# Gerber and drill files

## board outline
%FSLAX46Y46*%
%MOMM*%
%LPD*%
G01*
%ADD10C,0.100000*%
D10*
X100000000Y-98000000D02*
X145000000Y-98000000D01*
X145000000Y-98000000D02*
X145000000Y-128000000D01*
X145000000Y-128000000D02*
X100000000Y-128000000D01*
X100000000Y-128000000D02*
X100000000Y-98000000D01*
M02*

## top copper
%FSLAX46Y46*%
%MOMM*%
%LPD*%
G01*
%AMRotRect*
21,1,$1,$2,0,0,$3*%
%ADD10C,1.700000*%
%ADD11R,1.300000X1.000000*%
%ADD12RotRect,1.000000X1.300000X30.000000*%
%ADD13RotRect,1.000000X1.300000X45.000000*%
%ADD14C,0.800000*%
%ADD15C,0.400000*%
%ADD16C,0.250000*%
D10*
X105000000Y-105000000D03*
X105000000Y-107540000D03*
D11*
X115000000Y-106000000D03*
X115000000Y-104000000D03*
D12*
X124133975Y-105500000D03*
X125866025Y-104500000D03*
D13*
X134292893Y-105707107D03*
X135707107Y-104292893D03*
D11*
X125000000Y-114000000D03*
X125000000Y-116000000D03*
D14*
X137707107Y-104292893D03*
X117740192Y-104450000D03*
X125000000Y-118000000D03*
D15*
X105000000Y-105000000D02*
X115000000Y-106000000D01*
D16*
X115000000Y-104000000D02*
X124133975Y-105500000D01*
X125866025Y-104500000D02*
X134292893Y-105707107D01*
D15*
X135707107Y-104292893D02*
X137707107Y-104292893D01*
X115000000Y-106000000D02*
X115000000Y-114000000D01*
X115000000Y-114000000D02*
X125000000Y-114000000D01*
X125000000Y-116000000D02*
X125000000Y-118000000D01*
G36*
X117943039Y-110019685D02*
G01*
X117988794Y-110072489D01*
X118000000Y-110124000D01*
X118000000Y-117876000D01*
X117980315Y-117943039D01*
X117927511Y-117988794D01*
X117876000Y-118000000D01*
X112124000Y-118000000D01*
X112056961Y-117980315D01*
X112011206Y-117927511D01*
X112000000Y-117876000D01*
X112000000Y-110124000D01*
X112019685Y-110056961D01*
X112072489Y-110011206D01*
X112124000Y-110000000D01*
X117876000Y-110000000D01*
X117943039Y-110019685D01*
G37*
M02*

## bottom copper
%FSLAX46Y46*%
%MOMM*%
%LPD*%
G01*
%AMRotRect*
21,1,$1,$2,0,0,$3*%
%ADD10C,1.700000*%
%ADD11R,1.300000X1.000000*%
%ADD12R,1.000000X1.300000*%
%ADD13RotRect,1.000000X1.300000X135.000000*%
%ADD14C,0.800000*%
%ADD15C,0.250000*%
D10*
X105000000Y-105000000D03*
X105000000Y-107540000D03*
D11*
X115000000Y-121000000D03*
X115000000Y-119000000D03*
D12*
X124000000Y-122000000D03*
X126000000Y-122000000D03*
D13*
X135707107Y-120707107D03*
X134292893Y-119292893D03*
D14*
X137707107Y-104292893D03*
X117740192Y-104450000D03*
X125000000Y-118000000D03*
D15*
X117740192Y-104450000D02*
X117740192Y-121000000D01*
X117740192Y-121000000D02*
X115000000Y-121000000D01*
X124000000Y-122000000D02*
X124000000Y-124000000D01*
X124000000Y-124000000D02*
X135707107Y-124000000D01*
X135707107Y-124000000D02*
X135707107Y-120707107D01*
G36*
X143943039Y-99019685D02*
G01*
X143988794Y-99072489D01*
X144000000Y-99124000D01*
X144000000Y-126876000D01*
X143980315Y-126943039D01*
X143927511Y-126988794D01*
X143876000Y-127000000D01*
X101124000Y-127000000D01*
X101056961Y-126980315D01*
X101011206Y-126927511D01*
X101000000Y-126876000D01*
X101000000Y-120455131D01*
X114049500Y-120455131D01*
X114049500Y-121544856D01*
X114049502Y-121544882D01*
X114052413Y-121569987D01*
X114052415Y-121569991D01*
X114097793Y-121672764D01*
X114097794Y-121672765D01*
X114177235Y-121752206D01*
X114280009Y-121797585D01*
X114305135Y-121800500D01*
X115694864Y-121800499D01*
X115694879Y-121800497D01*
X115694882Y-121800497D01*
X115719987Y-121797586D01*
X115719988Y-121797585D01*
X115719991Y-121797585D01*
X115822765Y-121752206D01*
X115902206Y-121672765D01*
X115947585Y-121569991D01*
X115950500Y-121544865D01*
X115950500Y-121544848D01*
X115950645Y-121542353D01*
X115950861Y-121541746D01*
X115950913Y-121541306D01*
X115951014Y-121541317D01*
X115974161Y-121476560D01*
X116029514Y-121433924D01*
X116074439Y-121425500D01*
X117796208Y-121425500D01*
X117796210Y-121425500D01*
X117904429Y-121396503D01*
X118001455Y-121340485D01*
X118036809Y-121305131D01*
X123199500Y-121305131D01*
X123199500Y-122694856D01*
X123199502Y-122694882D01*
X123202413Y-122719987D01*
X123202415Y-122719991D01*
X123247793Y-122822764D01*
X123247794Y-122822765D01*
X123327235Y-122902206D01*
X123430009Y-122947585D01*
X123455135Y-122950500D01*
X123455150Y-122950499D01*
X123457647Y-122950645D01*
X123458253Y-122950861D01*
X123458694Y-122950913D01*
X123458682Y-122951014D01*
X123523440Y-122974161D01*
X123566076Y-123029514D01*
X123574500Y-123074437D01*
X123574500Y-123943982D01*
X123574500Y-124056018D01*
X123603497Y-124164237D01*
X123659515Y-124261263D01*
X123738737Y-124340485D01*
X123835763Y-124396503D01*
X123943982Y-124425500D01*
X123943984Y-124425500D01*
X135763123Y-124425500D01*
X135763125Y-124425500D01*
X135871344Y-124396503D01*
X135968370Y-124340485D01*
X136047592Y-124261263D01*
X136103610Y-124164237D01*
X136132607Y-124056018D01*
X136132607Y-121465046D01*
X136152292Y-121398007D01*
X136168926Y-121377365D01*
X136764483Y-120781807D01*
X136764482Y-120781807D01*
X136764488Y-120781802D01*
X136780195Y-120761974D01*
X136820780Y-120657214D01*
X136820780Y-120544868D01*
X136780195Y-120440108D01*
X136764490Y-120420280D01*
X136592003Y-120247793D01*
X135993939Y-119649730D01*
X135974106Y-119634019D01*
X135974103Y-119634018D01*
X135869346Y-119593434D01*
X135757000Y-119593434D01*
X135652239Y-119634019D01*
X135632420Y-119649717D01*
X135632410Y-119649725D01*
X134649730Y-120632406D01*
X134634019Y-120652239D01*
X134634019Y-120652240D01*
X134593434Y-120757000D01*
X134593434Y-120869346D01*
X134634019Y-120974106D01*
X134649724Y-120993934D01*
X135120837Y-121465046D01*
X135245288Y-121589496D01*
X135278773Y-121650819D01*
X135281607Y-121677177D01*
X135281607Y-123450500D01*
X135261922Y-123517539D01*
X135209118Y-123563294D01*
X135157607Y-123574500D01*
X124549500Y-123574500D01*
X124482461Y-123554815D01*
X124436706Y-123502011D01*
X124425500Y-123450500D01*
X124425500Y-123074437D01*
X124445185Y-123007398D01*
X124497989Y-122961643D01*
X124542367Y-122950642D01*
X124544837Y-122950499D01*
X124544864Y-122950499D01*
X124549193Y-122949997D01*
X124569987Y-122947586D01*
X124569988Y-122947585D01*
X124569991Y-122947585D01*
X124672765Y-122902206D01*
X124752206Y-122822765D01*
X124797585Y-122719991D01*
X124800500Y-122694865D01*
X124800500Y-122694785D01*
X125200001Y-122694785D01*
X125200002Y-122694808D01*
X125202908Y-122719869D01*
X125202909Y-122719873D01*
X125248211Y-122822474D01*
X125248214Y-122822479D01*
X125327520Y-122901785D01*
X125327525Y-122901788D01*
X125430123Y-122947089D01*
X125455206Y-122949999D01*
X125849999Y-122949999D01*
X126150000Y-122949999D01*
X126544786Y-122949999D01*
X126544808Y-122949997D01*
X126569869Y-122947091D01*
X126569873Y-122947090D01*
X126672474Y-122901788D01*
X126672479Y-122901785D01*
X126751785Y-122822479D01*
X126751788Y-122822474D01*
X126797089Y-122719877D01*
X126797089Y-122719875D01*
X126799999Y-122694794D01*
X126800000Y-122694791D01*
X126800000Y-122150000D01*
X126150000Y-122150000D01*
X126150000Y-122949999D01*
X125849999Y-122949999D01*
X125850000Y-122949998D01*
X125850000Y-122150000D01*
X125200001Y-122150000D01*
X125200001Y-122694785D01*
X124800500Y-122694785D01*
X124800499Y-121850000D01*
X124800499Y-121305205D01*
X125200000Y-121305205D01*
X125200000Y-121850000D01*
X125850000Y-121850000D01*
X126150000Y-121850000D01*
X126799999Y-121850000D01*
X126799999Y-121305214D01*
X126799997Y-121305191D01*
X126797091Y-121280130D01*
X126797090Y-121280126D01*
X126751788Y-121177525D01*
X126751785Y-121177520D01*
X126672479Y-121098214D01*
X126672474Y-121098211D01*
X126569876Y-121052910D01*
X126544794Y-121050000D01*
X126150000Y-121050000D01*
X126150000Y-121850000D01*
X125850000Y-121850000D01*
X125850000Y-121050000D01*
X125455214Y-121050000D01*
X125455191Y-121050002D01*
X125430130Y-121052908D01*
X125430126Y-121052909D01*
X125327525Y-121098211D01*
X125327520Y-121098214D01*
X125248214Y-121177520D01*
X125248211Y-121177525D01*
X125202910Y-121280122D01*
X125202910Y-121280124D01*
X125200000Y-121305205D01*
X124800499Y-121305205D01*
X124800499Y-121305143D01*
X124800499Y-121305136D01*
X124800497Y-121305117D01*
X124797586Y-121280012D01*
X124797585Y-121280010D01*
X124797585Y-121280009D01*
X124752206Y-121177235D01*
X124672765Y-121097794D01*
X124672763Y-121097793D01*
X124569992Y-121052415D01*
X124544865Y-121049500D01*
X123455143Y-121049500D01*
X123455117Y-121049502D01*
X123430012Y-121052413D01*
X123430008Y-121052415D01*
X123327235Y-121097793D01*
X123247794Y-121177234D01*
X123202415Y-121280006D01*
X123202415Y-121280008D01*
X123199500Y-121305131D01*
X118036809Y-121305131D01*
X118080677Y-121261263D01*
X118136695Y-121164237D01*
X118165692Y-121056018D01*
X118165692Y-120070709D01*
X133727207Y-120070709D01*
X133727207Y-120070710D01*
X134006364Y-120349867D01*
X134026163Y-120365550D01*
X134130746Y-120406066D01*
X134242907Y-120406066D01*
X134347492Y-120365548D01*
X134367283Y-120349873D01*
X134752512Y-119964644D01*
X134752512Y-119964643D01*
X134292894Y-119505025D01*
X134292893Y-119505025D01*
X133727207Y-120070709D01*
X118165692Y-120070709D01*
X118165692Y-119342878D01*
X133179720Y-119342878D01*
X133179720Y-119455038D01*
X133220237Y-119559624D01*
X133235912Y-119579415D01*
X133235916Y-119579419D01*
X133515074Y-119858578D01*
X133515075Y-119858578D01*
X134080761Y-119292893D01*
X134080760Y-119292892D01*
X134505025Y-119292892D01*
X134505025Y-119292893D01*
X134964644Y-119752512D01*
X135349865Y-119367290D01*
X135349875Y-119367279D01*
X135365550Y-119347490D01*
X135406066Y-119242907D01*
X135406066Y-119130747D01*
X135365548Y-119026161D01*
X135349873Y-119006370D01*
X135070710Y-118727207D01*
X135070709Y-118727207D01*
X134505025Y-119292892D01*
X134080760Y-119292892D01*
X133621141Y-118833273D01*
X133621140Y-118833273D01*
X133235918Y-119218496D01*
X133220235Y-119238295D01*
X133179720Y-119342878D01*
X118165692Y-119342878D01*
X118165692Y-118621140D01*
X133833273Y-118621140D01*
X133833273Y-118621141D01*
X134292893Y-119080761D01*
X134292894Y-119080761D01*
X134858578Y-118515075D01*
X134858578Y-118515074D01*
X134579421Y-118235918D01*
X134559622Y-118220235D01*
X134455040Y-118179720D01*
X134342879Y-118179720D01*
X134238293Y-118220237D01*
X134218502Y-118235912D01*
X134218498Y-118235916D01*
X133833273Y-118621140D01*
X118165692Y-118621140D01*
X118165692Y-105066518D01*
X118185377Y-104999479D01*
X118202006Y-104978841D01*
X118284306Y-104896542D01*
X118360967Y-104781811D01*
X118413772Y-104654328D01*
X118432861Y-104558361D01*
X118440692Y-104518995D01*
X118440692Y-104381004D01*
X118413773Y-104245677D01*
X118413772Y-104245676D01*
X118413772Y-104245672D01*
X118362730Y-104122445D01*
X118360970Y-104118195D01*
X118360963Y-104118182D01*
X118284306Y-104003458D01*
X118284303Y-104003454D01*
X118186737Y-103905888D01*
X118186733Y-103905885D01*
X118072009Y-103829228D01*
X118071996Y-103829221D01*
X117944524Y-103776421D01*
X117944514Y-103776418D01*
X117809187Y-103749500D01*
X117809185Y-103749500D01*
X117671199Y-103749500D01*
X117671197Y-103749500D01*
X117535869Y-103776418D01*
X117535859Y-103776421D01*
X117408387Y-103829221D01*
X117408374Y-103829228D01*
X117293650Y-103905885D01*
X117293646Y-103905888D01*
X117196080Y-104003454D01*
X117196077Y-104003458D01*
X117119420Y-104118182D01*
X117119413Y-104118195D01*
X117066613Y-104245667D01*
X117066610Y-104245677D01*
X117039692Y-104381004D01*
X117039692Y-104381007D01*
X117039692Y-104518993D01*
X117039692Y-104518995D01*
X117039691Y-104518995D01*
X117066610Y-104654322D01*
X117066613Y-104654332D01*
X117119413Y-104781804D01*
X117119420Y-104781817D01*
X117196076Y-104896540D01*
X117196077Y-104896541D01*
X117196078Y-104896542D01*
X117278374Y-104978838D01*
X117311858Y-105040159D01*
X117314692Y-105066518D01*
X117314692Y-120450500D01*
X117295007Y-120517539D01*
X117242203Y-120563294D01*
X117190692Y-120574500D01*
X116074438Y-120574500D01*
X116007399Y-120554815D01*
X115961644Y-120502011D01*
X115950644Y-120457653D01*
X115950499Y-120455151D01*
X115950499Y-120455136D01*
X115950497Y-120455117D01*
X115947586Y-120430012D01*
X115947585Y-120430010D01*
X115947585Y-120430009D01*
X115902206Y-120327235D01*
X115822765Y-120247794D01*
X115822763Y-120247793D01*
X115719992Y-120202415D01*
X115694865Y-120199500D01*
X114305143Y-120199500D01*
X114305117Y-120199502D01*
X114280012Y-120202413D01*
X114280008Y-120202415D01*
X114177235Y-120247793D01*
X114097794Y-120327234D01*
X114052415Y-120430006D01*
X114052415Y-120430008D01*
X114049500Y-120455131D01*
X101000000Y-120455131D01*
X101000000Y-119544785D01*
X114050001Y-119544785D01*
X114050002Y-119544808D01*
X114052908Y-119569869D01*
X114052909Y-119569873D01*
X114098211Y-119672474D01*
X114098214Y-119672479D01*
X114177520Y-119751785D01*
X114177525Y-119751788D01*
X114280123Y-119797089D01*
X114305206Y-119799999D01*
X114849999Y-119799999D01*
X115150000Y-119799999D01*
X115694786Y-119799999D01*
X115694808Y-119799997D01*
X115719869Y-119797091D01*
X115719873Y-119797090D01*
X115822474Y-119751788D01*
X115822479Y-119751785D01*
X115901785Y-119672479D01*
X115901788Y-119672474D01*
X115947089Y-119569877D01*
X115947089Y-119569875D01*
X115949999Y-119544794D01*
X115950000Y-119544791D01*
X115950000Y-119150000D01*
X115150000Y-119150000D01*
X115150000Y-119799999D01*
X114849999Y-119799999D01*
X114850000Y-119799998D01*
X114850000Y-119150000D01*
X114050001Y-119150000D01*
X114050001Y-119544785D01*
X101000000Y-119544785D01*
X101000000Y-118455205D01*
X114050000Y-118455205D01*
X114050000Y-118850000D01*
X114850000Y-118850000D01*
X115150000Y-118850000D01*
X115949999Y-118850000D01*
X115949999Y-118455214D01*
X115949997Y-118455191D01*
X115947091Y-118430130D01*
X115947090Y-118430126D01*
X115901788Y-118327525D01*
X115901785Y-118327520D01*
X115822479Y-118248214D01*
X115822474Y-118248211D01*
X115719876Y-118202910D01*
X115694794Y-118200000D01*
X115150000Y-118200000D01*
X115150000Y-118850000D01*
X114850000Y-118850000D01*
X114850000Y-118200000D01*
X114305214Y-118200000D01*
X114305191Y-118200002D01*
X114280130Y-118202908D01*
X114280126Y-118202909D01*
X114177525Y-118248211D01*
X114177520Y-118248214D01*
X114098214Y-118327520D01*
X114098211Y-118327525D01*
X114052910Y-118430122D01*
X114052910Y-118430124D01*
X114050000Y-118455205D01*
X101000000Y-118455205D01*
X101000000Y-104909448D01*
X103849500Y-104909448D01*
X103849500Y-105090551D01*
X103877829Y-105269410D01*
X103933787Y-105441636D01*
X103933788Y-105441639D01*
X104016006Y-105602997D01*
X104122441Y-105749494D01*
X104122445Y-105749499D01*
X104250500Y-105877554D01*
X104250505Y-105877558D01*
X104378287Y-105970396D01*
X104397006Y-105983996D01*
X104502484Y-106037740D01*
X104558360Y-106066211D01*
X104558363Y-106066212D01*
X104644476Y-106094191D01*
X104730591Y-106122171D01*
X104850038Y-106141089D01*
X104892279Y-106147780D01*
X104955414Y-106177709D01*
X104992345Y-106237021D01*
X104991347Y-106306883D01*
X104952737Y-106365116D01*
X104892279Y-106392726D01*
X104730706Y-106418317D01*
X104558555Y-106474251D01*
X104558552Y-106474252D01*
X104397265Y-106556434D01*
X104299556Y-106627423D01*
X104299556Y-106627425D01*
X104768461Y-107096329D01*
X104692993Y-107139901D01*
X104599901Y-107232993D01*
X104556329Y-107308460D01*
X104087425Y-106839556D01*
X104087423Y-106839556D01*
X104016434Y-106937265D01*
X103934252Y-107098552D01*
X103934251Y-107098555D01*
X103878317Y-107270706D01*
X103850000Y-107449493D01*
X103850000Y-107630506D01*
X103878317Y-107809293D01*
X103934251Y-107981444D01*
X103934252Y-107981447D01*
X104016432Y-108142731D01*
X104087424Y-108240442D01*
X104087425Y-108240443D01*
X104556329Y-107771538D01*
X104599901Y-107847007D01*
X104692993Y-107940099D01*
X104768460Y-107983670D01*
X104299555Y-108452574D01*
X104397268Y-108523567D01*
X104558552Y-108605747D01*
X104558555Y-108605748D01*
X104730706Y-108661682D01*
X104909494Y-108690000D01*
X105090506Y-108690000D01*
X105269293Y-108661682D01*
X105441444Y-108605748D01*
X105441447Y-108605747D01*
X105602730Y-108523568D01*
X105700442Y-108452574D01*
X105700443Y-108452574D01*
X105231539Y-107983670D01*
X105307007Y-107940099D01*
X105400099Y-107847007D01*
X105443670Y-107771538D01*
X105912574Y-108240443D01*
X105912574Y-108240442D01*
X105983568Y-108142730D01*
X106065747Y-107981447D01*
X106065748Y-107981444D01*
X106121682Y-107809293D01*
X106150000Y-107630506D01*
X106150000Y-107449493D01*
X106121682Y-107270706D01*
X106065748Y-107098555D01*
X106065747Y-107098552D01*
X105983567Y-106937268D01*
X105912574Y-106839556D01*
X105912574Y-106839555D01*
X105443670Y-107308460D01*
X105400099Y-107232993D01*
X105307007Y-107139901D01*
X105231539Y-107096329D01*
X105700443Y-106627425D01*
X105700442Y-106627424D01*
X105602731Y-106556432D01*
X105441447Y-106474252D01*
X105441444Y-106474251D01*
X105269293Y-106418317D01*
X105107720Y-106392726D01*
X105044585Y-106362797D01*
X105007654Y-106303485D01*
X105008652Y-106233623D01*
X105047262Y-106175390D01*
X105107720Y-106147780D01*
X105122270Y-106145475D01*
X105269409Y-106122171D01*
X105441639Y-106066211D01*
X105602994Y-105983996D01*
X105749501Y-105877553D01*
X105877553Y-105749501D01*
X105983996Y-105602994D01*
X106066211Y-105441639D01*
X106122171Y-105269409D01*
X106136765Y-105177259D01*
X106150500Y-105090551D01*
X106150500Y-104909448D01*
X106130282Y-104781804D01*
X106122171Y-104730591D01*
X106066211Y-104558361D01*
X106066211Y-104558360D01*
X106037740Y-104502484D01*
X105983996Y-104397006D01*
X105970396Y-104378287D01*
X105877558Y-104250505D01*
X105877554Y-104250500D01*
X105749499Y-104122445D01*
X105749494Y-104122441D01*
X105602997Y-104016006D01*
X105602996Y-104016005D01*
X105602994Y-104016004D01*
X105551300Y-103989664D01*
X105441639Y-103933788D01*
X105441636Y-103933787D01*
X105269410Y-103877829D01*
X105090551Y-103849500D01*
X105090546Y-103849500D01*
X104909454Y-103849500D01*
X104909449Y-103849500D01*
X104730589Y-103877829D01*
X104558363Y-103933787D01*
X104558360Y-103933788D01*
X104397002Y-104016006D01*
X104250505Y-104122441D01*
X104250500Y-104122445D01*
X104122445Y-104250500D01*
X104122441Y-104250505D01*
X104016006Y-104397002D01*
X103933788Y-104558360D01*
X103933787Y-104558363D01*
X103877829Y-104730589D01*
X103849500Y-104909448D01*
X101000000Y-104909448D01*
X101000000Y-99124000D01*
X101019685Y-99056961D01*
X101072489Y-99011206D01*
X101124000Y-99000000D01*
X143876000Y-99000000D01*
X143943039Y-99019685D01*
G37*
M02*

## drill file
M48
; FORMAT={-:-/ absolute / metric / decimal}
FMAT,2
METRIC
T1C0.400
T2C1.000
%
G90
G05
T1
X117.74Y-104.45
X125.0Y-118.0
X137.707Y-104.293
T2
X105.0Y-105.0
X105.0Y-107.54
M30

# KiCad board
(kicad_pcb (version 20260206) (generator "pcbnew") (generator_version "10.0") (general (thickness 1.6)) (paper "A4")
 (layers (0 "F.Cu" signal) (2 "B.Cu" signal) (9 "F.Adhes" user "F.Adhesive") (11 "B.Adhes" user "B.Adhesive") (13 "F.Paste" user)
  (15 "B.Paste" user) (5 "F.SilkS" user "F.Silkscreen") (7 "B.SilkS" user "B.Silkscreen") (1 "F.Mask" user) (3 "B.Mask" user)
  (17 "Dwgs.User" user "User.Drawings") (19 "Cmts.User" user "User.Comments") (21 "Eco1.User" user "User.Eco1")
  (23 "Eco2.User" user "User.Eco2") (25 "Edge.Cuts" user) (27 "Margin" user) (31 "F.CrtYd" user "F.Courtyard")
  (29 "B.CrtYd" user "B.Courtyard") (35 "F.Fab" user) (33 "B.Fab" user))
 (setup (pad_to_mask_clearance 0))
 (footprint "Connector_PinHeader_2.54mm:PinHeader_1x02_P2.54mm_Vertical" (layer "F.Cu") (at 105 105)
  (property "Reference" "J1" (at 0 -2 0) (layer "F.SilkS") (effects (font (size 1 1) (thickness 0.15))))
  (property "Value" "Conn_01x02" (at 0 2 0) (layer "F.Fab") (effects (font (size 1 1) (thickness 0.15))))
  (pad "1" thru_hole circle (at 0 0) (size 1.7 1.7) (drill 1) (layers "*.Cu" "*.Mask") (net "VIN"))
  (pad "2" thru_hole circle (at 0 2.54) (size 1.7 1.7) (drill 1) (layers "*.Cu" "*.Mask") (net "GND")))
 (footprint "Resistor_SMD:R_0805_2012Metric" (layer "F.Cu") (at 115 105 90)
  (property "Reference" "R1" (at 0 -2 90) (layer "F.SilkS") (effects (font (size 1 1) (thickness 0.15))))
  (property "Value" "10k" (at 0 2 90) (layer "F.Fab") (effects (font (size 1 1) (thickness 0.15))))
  (pad "1" smd rect (at -1 0 90) (size 1 1.3) (layers "F.Cu" "F.Paste" "F.Mask") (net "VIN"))
  (pad "2" smd rect (at 1 0 90) (size 1 1.3) (layers "F.Cu" "F.Paste" "F.Mask") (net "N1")))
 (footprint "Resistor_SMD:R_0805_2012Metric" (layer "F.Cu") (at 125 105 30)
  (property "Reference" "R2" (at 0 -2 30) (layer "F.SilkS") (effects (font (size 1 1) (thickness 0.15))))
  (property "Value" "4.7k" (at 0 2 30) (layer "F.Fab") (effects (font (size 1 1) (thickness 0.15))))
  (pad "1" smd rect (at -1 0 30) (size 1 1.3) (layers "F.Cu" "F.Paste" "F.Mask") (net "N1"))
  (pad "2" smd rect (at 1 0 30) (size 1 1.3) (layers "F.Cu" "F.Paste" "F.Mask") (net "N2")))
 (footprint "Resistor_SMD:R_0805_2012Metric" (layer "F.Cu") (at 135 105 45)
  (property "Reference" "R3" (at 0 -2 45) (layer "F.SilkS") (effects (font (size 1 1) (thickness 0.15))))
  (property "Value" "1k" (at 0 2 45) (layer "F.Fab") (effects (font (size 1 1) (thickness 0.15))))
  (pad "1" smd rect (at -1 0 45) (size 1 1.3) (layers "F.Cu" "F.Paste" "F.Mask") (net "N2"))
  (pad "2" smd rect (at 1 0 45) (size 1 1.3) (layers "F.Cu" "F.Paste" "F.Mask") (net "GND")))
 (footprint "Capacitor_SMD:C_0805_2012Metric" (layer "F.Cu") (at 125 115 270)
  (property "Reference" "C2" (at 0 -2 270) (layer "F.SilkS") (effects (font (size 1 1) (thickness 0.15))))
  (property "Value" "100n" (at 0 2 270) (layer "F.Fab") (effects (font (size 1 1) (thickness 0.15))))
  (pad "1" smd rect (at -1 0 270) (size 1 1.3) (layers "F.Cu" "F.Paste" "F.Mask") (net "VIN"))
  (pad "2" smd rect (at 1 0 270) (size 1 1.3) (layers "F.Cu" "F.Paste" "F.Mask") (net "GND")))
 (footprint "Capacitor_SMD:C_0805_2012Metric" (layer "B.Cu") (at 115 120 90)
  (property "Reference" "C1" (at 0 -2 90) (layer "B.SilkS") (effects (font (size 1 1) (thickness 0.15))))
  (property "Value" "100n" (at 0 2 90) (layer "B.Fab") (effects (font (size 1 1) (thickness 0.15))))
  (pad "1" smd rect (at -1 0 90) (size 1 1.3) (layers "B.Cu" "B.Paste" "B.Mask") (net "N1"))
  (pad "2" smd rect (at 1 0 90) (size 1 1.3) (layers "B.Cu" "B.Paste" "B.Mask") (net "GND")))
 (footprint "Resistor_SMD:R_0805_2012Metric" (layer "B.Cu") (at 125 122)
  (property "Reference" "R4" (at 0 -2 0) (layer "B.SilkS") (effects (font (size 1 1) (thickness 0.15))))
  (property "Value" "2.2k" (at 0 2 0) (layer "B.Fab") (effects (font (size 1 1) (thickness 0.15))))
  (pad "1" smd rect (at -1 0) (size 1 1.3) (layers "B.Cu" "B.Paste" "B.Mask") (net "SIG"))
  (pad "2" smd rect (at 1 0) (size 1 1.3) (layers "B.Cu" "B.Paste" "B.Mask") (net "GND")))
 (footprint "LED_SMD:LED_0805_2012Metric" (layer "B.Cu") (at 135 120 135)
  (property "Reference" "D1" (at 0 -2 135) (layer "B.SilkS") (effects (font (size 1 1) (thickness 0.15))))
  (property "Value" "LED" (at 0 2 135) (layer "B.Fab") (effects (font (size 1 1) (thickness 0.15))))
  (pad "1" smd rect (at -1 0 135) (size 1 1.3) (layers "B.Cu" "B.Paste" "B.Mask") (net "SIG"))
  (pad "2" smd rect (at 1 0 135) (size 1 1.3) (layers "B.Cu" "B.Paste" "B.Mask") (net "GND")))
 (gr_line (start 100 98) (end 145 98) (stroke (width 0.1) (type solid)) (layer "Edge.Cuts"))
 (gr_line (start 145 98) (end 145 128) (stroke (width 0.1) (type solid)) (layer "Edge.Cuts"))
 (gr_line (start 145 128) (end 100 128) (stroke (width 0.1) (type solid)) (layer "Edge.Cuts"))
 (gr_line (start 100 128) (end 100 98) (stroke (width 0.1) (type solid)) (layer "Edge.Cuts"))
 (segment (start 105 105) (end 115 106) (width 0.4) (layer "F.Cu") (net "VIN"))
 (segment (start 115 104) (end 124.133975 105.5) (width 0.25) (layer "F.Cu") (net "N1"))
 (segment (start 125.866025 104.5) (end 134.292893 105.707107) (width 0.25) (layer "F.Cu") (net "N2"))
 (segment (start 135.707107 104.292893) (end 137.707107 104.292893) (width 0.4) (layer "F.Cu") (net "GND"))
 (segment (start 115 106) (end 115 114) (width 0.4) (layer "F.Cu") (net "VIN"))
 (segment (start 115 114) (end 125 114) (width 0.4) (layer "F.Cu") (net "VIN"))
 (segment (start 117.740192 104.45) (end 117.740192 121) (width 0.25) (layer "B.Cu") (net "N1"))
 (segment (start 117.740192 121) (end 115 121) (width 0.25) (layer "B.Cu") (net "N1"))
 (segment (start 124 122) (end 124 124) (width 0.25) (layer "B.Cu") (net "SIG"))
 (segment (start 124 124) (end 135.707107 124) (width 0.25) (layer "B.Cu") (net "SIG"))
 (segment (start 135.707107 124) (end 135.707107 120.707107) (width 0.25) (layer "B.Cu") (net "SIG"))
 (segment (start 125 116) (end 125 118) (width 0.4) (layer "F.Cu") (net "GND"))
 (via (at 137.707107 104.292893) (size 0.8) (drill 0.4) (layers "F.Cu" "B.Cu") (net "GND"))
 (via (at 117.740192 104.45) (size 0.8) (drill 0.4) (layers "F.Cu" "B.Cu") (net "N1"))
 (via (at 125 118) (size 0.8) (drill 0.4) (layers "F.Cu" "B.Cu") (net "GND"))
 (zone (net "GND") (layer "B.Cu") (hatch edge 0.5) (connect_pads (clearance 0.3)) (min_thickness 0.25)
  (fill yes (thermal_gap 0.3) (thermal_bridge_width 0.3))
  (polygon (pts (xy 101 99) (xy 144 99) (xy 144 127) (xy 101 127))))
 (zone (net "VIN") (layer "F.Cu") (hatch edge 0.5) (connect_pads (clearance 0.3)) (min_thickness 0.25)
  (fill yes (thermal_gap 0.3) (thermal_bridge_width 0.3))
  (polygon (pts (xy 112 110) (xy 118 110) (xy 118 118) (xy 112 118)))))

